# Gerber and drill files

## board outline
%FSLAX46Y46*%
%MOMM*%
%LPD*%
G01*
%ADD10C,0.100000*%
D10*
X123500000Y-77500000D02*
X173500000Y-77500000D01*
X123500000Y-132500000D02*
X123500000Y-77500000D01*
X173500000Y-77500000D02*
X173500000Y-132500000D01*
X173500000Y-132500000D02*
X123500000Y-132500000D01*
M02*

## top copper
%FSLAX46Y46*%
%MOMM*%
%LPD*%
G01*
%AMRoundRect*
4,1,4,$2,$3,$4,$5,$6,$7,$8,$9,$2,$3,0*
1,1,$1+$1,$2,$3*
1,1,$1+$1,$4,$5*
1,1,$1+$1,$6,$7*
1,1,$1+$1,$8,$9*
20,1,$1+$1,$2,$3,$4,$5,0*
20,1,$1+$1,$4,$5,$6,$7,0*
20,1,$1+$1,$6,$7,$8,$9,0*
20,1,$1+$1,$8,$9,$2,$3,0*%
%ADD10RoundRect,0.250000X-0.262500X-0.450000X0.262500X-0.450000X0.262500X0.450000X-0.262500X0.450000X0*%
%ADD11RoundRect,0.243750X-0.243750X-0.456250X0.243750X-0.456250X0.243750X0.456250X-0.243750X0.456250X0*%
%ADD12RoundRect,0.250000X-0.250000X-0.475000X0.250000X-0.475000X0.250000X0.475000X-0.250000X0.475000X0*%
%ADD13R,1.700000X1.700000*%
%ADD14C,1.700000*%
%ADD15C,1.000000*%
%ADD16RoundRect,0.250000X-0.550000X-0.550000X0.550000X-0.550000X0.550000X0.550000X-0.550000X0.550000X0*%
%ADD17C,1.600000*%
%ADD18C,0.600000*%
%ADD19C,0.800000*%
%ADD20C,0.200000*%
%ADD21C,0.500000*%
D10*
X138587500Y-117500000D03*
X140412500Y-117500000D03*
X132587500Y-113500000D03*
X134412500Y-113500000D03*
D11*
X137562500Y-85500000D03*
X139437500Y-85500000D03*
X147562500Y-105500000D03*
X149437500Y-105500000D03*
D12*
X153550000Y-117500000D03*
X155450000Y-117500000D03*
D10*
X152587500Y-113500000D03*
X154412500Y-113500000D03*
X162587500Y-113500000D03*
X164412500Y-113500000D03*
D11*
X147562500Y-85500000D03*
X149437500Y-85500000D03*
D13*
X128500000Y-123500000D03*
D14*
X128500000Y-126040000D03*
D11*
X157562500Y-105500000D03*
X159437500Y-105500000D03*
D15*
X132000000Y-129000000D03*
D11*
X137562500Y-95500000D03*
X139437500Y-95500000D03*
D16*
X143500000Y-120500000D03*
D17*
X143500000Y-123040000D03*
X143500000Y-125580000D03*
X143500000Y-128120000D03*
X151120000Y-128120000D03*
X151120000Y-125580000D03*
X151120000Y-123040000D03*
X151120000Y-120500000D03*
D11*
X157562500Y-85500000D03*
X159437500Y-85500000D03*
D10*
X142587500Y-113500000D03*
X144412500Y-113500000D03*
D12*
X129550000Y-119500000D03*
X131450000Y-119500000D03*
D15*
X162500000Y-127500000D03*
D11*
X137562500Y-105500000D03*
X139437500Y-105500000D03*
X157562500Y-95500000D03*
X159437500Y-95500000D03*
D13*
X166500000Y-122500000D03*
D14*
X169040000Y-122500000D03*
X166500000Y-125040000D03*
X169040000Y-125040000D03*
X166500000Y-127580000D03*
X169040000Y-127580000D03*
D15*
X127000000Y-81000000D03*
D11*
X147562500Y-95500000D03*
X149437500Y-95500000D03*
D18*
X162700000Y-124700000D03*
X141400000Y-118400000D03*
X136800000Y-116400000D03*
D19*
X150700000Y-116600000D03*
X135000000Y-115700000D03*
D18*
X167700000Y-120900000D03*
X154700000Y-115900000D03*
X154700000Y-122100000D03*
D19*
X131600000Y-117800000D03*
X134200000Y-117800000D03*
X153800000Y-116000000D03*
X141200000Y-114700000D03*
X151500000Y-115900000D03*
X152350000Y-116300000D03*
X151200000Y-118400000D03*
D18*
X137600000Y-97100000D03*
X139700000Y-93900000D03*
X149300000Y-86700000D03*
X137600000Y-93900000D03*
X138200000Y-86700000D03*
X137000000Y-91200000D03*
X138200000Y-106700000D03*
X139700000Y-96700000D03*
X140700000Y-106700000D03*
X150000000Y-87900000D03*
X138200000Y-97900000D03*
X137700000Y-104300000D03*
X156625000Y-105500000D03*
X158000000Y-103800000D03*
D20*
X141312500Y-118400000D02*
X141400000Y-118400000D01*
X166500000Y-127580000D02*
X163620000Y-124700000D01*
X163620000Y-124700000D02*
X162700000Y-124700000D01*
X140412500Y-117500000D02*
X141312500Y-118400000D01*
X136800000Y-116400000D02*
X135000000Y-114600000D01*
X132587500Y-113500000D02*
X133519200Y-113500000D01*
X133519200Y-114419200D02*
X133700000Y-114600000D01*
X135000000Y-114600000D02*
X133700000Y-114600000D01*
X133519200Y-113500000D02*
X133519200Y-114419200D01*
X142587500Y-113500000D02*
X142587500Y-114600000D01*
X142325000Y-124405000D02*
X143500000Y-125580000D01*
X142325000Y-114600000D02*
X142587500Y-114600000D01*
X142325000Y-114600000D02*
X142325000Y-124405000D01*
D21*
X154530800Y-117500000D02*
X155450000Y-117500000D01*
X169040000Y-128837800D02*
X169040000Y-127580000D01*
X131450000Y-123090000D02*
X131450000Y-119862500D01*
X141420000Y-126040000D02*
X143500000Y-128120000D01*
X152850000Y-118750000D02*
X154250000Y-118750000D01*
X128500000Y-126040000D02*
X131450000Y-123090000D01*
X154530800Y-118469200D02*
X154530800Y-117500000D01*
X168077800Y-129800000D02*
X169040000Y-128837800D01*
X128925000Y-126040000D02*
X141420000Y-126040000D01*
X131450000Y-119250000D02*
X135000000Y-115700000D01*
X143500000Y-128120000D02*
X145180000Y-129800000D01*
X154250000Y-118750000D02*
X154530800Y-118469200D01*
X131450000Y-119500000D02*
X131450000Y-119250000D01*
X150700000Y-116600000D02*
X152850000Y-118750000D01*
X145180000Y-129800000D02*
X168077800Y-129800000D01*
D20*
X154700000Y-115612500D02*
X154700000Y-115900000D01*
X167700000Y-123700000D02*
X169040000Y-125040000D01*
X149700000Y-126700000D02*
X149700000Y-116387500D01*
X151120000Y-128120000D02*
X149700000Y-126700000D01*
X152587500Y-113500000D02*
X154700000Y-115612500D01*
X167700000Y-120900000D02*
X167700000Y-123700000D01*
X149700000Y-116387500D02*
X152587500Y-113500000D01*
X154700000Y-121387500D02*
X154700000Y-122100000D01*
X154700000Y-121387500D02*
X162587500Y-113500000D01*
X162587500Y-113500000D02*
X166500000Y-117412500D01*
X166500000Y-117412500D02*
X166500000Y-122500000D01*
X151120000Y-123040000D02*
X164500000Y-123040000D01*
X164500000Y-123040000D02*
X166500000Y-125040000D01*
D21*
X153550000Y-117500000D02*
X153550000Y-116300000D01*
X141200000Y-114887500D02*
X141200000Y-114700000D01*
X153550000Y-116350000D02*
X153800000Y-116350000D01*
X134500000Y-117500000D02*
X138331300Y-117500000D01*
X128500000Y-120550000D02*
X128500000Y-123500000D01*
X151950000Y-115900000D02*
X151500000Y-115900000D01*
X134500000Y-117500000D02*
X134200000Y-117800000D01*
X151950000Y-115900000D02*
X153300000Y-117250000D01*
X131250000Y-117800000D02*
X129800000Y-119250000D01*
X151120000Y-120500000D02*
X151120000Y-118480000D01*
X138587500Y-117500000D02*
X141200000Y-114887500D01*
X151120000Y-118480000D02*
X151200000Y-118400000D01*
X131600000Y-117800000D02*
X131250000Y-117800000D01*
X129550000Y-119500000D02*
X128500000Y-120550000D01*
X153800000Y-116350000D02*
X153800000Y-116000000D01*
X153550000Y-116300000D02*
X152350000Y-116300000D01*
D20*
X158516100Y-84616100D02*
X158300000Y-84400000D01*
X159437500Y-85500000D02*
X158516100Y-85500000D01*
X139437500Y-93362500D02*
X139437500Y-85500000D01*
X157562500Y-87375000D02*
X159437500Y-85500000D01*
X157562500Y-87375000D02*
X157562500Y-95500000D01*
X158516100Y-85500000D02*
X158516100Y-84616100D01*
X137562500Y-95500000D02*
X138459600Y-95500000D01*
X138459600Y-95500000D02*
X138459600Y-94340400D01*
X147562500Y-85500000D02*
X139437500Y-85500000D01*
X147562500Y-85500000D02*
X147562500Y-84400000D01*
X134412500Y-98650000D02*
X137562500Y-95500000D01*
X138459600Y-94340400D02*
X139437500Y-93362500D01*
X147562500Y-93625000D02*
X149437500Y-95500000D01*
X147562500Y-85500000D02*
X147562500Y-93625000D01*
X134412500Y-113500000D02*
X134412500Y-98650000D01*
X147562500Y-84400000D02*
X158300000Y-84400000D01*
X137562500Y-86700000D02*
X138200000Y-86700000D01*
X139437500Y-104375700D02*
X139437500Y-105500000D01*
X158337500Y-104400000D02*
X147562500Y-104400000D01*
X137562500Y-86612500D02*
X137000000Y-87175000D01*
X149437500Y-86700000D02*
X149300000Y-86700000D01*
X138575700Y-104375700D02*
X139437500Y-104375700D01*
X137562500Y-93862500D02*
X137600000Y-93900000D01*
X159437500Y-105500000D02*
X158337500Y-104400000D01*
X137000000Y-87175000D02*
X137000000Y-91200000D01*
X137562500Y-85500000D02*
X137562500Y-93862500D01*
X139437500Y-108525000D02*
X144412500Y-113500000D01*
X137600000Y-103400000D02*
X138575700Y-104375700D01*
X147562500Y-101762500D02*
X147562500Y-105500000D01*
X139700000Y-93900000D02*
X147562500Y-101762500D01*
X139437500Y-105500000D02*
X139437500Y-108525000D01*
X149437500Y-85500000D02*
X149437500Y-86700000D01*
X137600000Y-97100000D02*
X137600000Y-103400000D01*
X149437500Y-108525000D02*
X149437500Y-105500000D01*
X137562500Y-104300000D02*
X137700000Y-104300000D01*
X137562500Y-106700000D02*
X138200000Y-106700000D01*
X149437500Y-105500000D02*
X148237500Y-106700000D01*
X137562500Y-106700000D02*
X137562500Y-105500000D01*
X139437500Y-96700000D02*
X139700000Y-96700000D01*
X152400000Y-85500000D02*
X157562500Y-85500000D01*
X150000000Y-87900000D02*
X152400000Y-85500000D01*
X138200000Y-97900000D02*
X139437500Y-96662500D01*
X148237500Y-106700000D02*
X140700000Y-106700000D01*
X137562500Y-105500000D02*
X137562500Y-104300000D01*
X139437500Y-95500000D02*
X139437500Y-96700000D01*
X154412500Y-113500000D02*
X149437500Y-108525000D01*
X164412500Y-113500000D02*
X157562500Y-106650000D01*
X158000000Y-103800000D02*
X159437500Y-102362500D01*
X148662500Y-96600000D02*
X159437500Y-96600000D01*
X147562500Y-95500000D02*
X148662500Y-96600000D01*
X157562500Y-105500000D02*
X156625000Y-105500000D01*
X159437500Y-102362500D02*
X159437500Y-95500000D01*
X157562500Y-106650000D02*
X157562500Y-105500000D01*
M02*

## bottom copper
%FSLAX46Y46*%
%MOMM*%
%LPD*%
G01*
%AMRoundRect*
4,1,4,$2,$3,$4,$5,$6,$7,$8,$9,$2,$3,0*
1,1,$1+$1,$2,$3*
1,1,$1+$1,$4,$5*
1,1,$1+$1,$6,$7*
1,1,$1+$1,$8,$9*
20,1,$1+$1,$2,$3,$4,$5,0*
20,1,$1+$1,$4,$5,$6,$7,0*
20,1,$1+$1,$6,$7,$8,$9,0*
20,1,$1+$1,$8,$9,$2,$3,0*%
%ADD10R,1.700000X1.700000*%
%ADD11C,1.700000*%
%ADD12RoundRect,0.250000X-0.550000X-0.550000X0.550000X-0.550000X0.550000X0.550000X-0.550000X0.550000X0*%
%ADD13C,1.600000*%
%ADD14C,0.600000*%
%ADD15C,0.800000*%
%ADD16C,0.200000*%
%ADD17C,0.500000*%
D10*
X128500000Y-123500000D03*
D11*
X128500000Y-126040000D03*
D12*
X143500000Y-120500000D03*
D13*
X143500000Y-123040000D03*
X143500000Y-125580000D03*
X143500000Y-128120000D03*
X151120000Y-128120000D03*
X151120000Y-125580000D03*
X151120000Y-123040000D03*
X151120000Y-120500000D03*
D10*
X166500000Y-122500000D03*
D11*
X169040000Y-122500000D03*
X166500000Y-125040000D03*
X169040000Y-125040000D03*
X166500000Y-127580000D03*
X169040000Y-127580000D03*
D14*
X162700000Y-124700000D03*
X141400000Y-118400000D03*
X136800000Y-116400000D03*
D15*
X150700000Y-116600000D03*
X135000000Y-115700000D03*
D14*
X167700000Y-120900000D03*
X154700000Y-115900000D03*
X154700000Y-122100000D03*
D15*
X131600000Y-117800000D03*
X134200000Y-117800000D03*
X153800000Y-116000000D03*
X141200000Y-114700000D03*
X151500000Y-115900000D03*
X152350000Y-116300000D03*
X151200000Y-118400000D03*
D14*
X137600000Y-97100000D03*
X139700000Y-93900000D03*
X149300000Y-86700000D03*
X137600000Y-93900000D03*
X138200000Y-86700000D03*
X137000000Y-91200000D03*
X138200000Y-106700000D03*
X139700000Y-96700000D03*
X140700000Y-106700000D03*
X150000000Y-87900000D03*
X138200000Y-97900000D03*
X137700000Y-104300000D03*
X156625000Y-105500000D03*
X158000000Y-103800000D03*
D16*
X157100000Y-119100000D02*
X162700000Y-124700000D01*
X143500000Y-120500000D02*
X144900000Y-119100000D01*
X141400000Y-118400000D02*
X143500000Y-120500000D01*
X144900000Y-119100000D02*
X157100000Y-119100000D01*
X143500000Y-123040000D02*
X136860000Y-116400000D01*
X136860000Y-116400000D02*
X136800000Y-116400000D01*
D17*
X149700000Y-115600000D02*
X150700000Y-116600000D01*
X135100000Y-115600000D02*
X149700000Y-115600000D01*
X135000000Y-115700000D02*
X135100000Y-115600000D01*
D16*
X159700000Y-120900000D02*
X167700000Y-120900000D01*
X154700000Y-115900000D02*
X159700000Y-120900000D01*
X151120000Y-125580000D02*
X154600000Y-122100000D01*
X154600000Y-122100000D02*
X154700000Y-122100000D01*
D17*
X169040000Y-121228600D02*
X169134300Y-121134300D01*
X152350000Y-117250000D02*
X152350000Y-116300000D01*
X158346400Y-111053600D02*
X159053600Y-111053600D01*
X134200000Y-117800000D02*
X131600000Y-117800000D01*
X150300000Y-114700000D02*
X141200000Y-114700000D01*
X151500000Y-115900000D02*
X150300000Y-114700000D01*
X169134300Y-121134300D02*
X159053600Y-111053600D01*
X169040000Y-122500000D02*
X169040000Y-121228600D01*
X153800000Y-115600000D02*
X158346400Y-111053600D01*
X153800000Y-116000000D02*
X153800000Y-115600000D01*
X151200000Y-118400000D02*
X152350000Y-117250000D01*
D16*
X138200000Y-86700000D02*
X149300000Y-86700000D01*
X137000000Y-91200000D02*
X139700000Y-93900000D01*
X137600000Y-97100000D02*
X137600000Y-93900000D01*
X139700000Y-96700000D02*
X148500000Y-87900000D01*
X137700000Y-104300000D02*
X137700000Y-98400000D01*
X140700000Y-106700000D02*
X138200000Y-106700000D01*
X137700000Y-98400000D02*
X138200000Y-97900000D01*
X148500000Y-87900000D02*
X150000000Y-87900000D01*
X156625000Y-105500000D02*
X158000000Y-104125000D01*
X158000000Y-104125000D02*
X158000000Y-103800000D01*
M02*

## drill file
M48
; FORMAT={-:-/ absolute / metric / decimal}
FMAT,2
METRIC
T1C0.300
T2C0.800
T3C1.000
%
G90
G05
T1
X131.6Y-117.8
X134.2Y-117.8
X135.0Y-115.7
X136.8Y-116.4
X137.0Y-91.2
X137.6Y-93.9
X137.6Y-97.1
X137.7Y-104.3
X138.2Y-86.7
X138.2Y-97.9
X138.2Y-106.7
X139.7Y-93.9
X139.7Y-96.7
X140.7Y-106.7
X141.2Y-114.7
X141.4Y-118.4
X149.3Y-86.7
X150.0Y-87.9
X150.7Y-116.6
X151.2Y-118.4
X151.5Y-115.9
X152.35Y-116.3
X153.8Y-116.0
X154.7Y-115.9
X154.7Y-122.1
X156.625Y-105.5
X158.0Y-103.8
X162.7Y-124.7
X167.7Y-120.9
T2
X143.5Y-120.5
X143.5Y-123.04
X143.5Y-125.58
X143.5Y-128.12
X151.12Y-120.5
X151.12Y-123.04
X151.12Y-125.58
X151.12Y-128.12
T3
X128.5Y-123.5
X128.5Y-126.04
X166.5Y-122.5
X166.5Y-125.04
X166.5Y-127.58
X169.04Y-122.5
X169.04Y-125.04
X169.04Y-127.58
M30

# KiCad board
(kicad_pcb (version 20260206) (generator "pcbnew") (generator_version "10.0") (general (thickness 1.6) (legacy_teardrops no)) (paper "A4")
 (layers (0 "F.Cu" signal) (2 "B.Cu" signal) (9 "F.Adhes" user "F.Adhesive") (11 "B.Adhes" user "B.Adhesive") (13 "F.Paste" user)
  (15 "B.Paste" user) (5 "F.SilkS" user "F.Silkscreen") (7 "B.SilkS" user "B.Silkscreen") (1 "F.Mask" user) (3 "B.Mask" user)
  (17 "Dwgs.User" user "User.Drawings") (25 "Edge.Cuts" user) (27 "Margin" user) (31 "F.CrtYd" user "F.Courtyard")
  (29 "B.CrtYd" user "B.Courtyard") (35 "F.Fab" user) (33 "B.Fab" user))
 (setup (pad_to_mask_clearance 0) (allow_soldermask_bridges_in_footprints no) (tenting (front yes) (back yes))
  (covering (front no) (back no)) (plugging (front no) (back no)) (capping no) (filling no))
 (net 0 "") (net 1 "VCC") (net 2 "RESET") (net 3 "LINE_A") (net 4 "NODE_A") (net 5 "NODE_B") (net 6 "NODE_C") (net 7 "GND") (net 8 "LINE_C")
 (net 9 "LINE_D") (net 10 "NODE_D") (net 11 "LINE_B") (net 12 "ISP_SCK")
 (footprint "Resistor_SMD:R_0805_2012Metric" (layer "F.Cu") (at 139.5 117.5)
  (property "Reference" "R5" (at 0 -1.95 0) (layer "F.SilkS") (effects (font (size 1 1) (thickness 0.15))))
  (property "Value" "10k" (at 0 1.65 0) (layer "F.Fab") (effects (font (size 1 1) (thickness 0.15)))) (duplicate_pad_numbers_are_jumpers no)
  (pad "1" smd roundrect (at -0.9125 0) (size 1.025 1.4) (layers "F.Cu" "F.Mask" "F.Paste") (roundrect_rratio 0.243902) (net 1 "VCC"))
  (pad "2" smd roundrect (at 0.9125 0) (size 1.025 1.4) (layers "F.Cu" "F.Mask" "F.Paste") (roundrect_rratio 0.243902) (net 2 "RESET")))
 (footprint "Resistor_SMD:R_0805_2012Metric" (layer "F.Cu") (at 133.5 113.5)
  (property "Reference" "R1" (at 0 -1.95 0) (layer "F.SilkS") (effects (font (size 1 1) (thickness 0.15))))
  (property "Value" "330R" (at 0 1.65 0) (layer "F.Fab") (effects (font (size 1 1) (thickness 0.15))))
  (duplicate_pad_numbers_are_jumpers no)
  (pad "1" smd roundrect (at -0.9125 0) (size 1.025 1.4) (layers "F.Cu" "F.Mask" "F.Paste") (roundrect_rratio 0.243902) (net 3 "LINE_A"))
  (pad "2" smd roundrect (at 0.9125 0) (size 1.025 1.4) (layers "F.Cu" "F.Mask" "F.Paste") (roundrect_rratio 0.243902) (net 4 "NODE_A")))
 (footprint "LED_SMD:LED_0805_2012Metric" (layer "F.Cu") (at 138.5 85.5)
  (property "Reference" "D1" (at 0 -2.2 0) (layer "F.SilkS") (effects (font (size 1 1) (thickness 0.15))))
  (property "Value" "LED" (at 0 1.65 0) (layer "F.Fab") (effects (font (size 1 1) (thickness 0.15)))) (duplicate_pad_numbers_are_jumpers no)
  (pad "1" smd roundrect (at -0.9375 0) (size 0.975 1.4) (layers "F.Cu" "F.Mask" "F.Paste") (roundrect_rratio 0.25) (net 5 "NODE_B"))
  (pad "2" smd roundrect (at 0.9375 0) (size 0.975 1.4) (layers "F.Cu" "F.Mask" "F.Paste") (roundrect_rratio 0.25) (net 4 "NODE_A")))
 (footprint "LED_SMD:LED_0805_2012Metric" (layer "F.Cu") (at 148.5 105.5)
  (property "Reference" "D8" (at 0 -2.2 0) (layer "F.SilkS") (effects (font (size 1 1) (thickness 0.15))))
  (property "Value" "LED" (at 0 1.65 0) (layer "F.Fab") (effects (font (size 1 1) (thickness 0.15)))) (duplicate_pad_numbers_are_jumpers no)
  (pad "1" smd roundrect (at -0.9375 0) (size 0.975 1.4) (layers "F.Cu" "F.Mask" "F.Paste") (roundrect_rratio 0.25) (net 5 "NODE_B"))
  (pad "2" smd roundrect (at 0.9375 0) (size 0.975 1.4) (layers "F.Cu" "F.Mask" "F.Paste") (roundrect_rratio 0.25) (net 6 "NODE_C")))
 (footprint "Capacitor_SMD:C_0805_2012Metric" (layer "F.Cu") (at 154.5 117.5)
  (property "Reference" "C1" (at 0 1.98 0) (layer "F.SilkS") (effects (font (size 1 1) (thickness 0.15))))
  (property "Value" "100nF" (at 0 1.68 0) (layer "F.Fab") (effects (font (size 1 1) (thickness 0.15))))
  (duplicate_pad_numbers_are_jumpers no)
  (pad "1" smd roundrect (at -0.95 0) (size 1 1.45) (layers "F.Cu" "F.Mask" "F.Paste") (roundrect_rratio 0.25) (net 1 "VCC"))
  (pad "2" smd roundrect (at 0.95 0) (size 1 1.45) (layers "F.Cu" "F.Mask" "F.Paste") (roundrect_rratio 0.25) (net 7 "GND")))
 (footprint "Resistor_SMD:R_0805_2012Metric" (layer "F.Cu") (at 153.5 113.5)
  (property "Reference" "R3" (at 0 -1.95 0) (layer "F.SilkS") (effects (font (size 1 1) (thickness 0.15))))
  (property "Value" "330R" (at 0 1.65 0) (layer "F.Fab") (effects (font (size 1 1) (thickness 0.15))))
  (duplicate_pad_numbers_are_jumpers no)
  (pad "1" smd roundrect (at -0.9125 0) (size 1.025 1.4) (layers "F.Cu" "F.Mask" "F.Paste") (roundrect_rratio 0.243902) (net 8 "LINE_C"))
  (pad "2" smd roundrect (at 0.9125 0) (size 1.025 1.4) (layers "F.Cu" "F.Mask" "F.Paste") (roundrect_rratio 0.243902) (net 6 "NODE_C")))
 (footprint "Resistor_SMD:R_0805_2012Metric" (layer "F.Cu") (at 163.5 113.5)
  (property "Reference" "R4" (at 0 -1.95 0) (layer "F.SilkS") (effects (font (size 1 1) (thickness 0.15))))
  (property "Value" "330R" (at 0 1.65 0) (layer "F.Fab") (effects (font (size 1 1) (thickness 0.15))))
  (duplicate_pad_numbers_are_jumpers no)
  (pad "1" smd roundrect (at -0.9125 0) (size 1.025 1.4) (layers "F.Cu" "F.Mask" "F.Paste") (roundrect_rratio 0.243902) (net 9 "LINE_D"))
  (pad "2" smd roundrect (at 0.9125 0) (size 1.025 1.4) (layers "F.Cu" "F.Mask" "F.Paste") (roundrect_rratio 0.243902) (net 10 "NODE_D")))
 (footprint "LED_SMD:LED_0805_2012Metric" (layer "F.Cu") (at 148.5 85.5)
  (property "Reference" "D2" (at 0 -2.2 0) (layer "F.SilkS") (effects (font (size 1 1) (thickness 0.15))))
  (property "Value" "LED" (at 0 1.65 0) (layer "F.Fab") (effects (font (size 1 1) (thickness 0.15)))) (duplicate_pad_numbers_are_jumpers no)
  (pad "1" smd roundrect (at -0.9375 0) (size 0.975 1.4) (layers "F.Cu" "F.Mask" "F.Paste") (roundrect_rratio 0.25) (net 4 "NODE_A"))
  (pad "2" smd roundrect (at 0.9375 0) (size 0.975 1.4) (layers "F.Cu" "F.Mask" "F.Paste") (roundrect_rratio 0.25) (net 5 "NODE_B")))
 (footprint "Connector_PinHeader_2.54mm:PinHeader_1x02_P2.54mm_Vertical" (layer "F.Cu") (at 128.5 123.5)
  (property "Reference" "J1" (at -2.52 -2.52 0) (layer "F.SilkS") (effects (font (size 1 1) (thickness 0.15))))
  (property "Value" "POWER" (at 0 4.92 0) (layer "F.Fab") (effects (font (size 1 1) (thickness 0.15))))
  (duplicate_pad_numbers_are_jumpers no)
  (pad "1" thru_hole rect (at 0 0) (size 1.7 1.7) (drill 1) (layers "*.Cu" "*.Mask") (remove_unused_layers no) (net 1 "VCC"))
  (pad "2" thru_hole circle (at 0 2.54) (size 1.7 1.7) (drill 1) (layers "*.Cu" "*.Mask") (remove_unused_layers no) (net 7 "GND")))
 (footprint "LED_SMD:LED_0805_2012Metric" (layer "F.Cu") (at 158.5 105.5)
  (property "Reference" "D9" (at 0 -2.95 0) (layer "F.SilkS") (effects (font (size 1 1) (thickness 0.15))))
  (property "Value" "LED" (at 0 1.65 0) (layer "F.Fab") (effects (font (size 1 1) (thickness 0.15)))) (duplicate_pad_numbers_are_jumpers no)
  (pad "1" smd roundrect (at -0.9375 0) (size 0.975 1.4) (layers "F.Cu" "F.Mask" "F.Paste") (roundrect_rratio 0.25) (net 10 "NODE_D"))
  (pad "2" smd roundrect (at 0.9375 0) (size 0.975 1.4) (layers "F.Cu" "F.Mask" "F.Paste") (roundrect_rratio 0.25) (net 5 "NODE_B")))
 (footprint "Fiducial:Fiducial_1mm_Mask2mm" (layer "F.Cu") (at 132 129)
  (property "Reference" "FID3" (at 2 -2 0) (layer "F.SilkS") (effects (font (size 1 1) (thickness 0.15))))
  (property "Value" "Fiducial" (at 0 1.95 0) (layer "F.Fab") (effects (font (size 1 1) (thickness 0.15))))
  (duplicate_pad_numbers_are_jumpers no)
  (pad "" smd circle (at 0 0) (size 1 1) (layers "F.Cu" "F.Mask") (solder_mask_margin 0.5) (clearance 0.6)))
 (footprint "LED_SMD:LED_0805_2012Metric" (layer "F.Cu") (at 138.5 95.5)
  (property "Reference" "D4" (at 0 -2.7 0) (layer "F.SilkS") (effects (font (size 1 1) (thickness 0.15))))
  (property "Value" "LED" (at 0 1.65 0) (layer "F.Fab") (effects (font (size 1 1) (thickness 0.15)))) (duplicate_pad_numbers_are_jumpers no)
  (pad "1" smd roundrect (at -0.9375 0) (size 0.975 1.4) (layers "F.Cu" "F.Mask" "F.Paste") (roundrect_rratio 0.25) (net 4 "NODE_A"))
  (pad "2" smd roundrect (at 0.9375 0) (size 0.975 1.4) (layers "F.Cu" "F.Mask" "F.Paste") (roundrect_rratio 0.25) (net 6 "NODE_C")))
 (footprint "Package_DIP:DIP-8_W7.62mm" (layer "F.Cu") (at 143.5 120.5)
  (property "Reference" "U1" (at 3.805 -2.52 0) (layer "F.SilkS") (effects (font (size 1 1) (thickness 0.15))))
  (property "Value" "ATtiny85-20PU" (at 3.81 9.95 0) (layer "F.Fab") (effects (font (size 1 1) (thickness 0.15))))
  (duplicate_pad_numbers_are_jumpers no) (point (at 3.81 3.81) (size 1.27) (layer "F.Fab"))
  (pad "1" thru_hole roundrect (at 0 0) (size 1.6 1.6) (drill 0.8) (layers "*.Cu" "*.Mask") (remove_unused_layers no)
   (roundrect_rratio 0.15625) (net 2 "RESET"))
  (pad "2" thru_hole circle (at 0 2.54) (size 1.6 1.6) (drill 0.8) (layers "*.Cu" "*.Mask") (remove_unused_layers no) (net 3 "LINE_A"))
  (pad "3" thru_hole circle (at 0 5.08) (size 1.6 1.6) (drill 0.8) (layers "*.Cu" "*.Mask") (remove_unused_layers no) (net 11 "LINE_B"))
  (pad "4" thru_hole circle (at 0 7.62) (size 1.6 1.6) (drill 0.8) (layers "*.Cu" "*.Mask") (remove_unused_layers no) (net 7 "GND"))
  (pad "5" thru_hole circle (at 7.62 7.62) (size 1.6 1.6) (drill 0.8) (layers "*.Cu" "*.Mask") (remove_unused_layers no) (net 8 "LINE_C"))
  (pad "6" thru_hole circle (at 7.62 5.08) (size 1.6 1.6) (drill 0.8) (layers "*.Cu" "*.Mask") (remove_unused_layers no) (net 9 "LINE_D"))
  (pad "7" thru_hole circle (at 7.62 2.54) (size 1.6 1.6) (drill 0.8) (layers "*.Cu" "*.Mask") (remove_unused_layers no) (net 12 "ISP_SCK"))
  (pad "8" thru_hole circle (at 7.62 0) (size 1.6 1.6) (drill 0.8) (layers "*.Cu" "*.Mask") (remove_unused_layers no) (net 1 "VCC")))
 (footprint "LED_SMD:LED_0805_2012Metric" (layer "F.Cu") (at 158.5 85.5)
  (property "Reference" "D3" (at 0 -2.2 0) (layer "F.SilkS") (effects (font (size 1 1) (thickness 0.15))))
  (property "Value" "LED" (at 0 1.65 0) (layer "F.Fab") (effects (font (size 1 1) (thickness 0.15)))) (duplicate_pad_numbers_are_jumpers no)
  (pad "1" smd roundrect (at -0.9375 0) (size 0.975 1.4) (layers "F.Cu" "F.Mask" "F.Paste") (roundrect_rratio 0.25) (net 6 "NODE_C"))
  (pad "2" smd roundrect (at 0.9375 0) (size 0.975 1.4) (layers "F.Cu" "F.Mask" "F.Paste") (roundrect_rratio 0.25) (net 4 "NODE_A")))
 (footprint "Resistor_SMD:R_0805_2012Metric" (layer "F.Cu") (at 143.5 113.5)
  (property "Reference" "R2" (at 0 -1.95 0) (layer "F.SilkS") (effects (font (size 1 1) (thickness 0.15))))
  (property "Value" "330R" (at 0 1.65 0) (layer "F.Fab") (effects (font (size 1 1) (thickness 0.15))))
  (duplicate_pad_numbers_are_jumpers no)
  (pad "1" smd roundrect (at -0.9125 0) (size 1.025 1.4) (layers "F.Cu" "F.Mask" "F.Paste") (roundrect_rratio 0.243902) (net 11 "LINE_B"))
  (pad "2" smd roundrect (at 0.9125 0) (size 1.025 1.4) (layers "F.Cu" "F.Mask" "F.Paste") (roundrect_rratio 0.243902) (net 5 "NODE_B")))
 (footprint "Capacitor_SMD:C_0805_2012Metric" (layer "F.Cu") (at 130.5 119.5)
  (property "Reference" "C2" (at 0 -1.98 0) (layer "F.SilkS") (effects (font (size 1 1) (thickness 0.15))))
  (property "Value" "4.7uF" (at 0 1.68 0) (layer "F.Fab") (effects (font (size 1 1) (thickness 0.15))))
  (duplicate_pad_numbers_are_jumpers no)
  (pad "1" smd roundrect (at -0.95 0) (size 1 1.45) (layers "F.Cu" "F.Mask" "F.Paste") (roundrect_rratio 0.25) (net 1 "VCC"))
  (pad "2" smd roundrect (at 0.95 0) (size 1 1.45) (layers "F.Cu" "F.Mask" "F.Paste") (roundrect_rratio 0.25) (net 7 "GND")))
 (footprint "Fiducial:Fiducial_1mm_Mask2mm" (layer "F.Cu") (at 162.5 127.5)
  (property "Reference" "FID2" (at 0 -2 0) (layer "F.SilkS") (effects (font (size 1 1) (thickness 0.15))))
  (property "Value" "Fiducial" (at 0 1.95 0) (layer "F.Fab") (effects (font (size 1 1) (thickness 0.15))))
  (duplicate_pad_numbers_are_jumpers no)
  (pad "" smd circle (at 0 0) (size 1 1) (layers "F.Cu" "F.Mask") (solder_mask_margin 0.5) (clearance 0.6)))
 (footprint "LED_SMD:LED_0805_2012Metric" (layer "F.Cu") (at 138.5 105.5)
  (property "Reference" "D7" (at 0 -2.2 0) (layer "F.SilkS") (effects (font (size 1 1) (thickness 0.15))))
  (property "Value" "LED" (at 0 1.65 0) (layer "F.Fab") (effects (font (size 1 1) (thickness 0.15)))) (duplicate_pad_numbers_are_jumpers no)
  (pad "1" smd roundrect (at -0.9375 0) (size 0.975 1.4) (layers "F.Cu" "F.Mask" "F.Paste") (roundrect_rratio 0.25) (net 6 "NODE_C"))
  (pad "2" smd roundrect (at 0.9375 0) (size 0.975 1.4) (layers "F.Cu" "F.Mask" "F.Paste") (roundrect_rratio 0.25) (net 5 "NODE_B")))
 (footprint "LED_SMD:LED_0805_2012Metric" (layer "F.Cu") (at 158.5 95.5)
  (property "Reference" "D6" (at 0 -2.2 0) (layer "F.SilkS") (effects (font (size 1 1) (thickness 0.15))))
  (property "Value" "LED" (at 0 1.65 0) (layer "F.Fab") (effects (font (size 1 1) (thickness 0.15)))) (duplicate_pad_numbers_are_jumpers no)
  (pad "1" smd roundrect (at -0.9375 0) (size 0.975 1.4) (layers "F.Cu" "F.Mask" "F.Paste") (roundrect_rratio 0.25) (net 4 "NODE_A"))
  (pad "2" smd roundrect (at 0.9375 0) (size 0.975 1.4) (layers "F.Cu" "F.Mask" "F.Paste") (roundrect_rratio 0.25) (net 10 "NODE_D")))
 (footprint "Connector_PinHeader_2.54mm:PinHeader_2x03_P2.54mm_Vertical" (layer "F.Cu") (at 166.5 122.5)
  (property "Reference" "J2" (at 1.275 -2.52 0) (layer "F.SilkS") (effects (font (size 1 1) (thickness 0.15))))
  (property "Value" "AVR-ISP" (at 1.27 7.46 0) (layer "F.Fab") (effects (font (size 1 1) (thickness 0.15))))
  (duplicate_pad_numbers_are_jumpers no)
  (pad "1" thru_hole rect (at 0 0) (size 1.7 1.7) (drill 1) (layers "*.Cu" "*.Mask") (remove_unused_layers no) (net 9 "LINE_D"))
  (pad "2" thru_hole circle (at 2.54 0) (size 1.7 1.7) (drill 1) (layers "*.Cu" "*.Mask") (remove_unused_layers no) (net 1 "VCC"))
  (pad "3" thru_hole circle (at 0 2.54) (size 1.7 1.7) (drill 1) (layers "*.Cu" "*.Mask") (remove_unused_layers no) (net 12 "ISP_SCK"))
  (pad "4" thru_hole circle (at 2.54 2.54) (size 1.7 1.7) (drill 1) (layers "*.Cu" "*.Mask") (remove_unused_layers no) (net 8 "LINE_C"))
  (pad "5" thru_hole circle (at 0 5.08) (size 1.7 1.7) (drill 1) (layers "*.Cu" "*.Mask") (remove_unused_layers no) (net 2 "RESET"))
  (pad "6" thru_hole circle (at 2.54 5.08) (size 1.7 1.7) (drill 1) (layers "*.Cu" "*.Mask") (remove_unused_layers no) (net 7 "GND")))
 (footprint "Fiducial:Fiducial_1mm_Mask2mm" (layer "F.Cu") (at 127 81)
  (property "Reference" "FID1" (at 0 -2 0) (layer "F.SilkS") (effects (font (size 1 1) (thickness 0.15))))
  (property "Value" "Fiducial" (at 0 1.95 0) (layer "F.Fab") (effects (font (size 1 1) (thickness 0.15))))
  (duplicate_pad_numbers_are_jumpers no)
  (pad "" smd circle (at 0 0) (size 1 1) (layers "F.Cu" "F.Mask") (solder_mask_margin 0.5) (clearance 0.6)))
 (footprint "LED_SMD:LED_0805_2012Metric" (layer "F.Cu") (at 148.5 95.5)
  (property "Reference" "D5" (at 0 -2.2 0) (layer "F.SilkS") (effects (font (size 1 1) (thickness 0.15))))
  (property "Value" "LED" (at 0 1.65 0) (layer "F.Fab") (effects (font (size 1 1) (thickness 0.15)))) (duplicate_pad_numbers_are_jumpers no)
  (pad "1" smd roundrect (at -0.9375 0) (size 0.975 1.4) (layers "F.Cu" "F.Mask" "F.Paste") (roundrect_rratio 0.25) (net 10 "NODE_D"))
  (pad "2" smd roundrect (at 0.9375 0) (size 0.975 1.4) (layers "F.Cu" "F.Mask" "F.Paste") (roundrect_rratio 0.25) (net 4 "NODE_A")))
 (gr_line (start 123.5 77.5) (end 173.5 77.5) (stroke (width 0.1) (type default)) (layer "Edge.Cuts"))
 (gr_line (start 123.5 132.5) (end 123.5 77.5) (stroke (width 0.1) (type default)) (layer "Edge.Cuts"))
 (gr_line (start 173.5 77.5) (end 173.5 132.5) (stroke (width 0.1) (type default)) (layer "Edge.Cuts"))
 (gr_line (start 173.5 132.5) (end 123.5 132.5) (stroke (width 0.1) (type default)) (layer "Edge.Cuts"))
 (segment (start 141.3125 118.4) (end 141.4 118.4) (width 0.2) (layer "F.Cu") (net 2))
 (segment (start 166.5 127.58) (end 163.62 124.7) (width 0.2) (layer "F.Cu") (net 2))
 (segment (start 163.62 124.7) (end 162.7 124.7) (width 0.2) (layer "F.Cu") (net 2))
 (segment (start 140.4125 117.5) (end 141.3125 118.4) (width 0.2) (layer "F.Cu") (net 2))
 (via (at 162.7 124.7) (size 0.6) (drill 0.3) (layers "F.Cu" "B.Cu") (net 2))
 (via (at 141.4 118.4) (size 0.6) (drill 0.3) (layers "F.Cu" "B.Cu") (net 2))
 (segment (start 157.1 119.1) (end 162.7 124.7) (width 0.2) (layer "B.Cu") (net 2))
 (segment (start 143.5 120.5) (end 144.9 119.1) (width 0.2) (layer "B.Cu") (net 2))
 (segment (start 141.4 118.4) (end 143.5 120.5) (width 0.2) (layer "B.Cu") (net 2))
 (segment (start 144.9 119.1) (end 157.1 119.1) (width 0.2) (layer "B.Cu") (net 2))
 (segment (start 136.8 116.4) (end 135 114.6) (width 0.2) (layer "F.Cu") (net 3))
 (segment (start 132.5875 113.5) (end 133.5192 113.5) (width 0.2) (layer "F.Cu") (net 3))
 (segment (start 133.5192 114.4192) (end 133.7 114.6) (width 0.2) (layer "F.Cu") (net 3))
 (segment (start 135 114.6) (end 133.7 114.6) (width 0.2) (layer "F.Cu") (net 3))
 (segment (start 133.5192 113.5) (end 133.5192 114.4192) (width 0.2) (layer "F.Cu") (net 3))
 (via (at 136.8 116.4) (size 0.6) (drill 0.3) (layers "F.Cu" "B.Cu") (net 3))
 (segment (start 143.5 123.04) (end 136.86 116.4) (width 0.2) (layer "B.Cu") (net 3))
 (segment (start 136.86 116.4) (end 136.8 116.4) (width 0.2) (layer "B.Cu") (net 3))
 (segment (start 142.5875 113.5) (end 142.5875 114.6) (width 0.2) (layer "F.Cu") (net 11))
 (segment (start 142.325 124.405) (end 143.5 125.58) (width 0.2) (layer "F.Cu") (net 11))
 (segment (start 142.325 114.6) (end 142.5875 114.6) (width 0.2) (layer "F.Cu") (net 11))
 (segment (start 142.325 114.6) (end 142.325 124.405) (width 0.2) (layer "F.Cu") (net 11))
 (segment (start 154.5308 117.5) (end 155.45 117.5) (width 0.5) (layer "F.Cu") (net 7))
 (segment (start 169.04 128.8378) (end 169.04 127.58) (width 0.5) (layer "F.Cu") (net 7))
 (segment (start 131.45 123.09) (end 131.45 119.8625) (width 0.5) (layer "F.Cu") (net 7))
 (segment (start 141.42 126.04) (end 143.5 128.12) (width 0.5) (layer "F.Cu") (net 7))
 (segment (start 152.85 118.75) (end 154.25 118.75) (width 0.5) (layer "F.Cu") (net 7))
 (segment (start 128.5 126.04) (end 131.45 123.09) (width 0.5) (layer "F.Cu") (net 7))
 (segment (start 154.5308 118.4692) (end 154.5308 117.5) (width 0.5) (layer "F.Cu") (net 7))
 (segment (start 168.0778 129.8) (end 169.04 128.8378) (width 0.5) (layer "F.Cu") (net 7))
 (segment (start 128.925 126.04) (end 141.42 126.04) (width 0.5) (layer "F.Cu") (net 7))
 (segment (start 131.45 119.25) (end 135 115.7) (width 0.5) (layer "F.Cu") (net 7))
 (segment (start 143.5 128.12) (end 145.18 129.8) (width 0.5) (layer "F.Cu") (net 7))
 (segment (start 154.25 118.75) (end 154.5308 118.4692) (width 0.5) (layer "F.Cu") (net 7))
 (segment (start 131.45 119.5) (end 131.45 119.25) (width 0.5) (layer "F.Cu") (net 7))
 (segment (start 150.7 116.6) (end 152.85 118.75) (width 0.5) (layer "F.Cu") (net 7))
 (segment (start 145.18 129.8) (end 168.0778 129.8) (width 0.5) (layer "F.Cu") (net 7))
 (via (at 150.7 116.6) (size 0.8) (drill 0.3) (layers "F.Cu" "B.Cu") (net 7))
 (via (at 135 115.7) (size 0.8) (drill 0.3) (layers "F.Cu" "B.Cu") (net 7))
 (segment (start 149.7 115.6) (end 150.7 116.6) (width 0.5) (layer "B.Cu") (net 7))
 (segment (start 135.1 115.6) (end 149.7 115.6) (width 0.5) (layer "B.Cu") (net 7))
 (segment (start 135 115.7) (end 135.1 115.6) (width 0.5) (layer "B.Cu") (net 7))
 (segment (start 154.7 115.6125) (end 154.7 115.9) (width 0.2) (layer "F.Cu") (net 8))
 (segment (start 167.7 123.7) (end 169.04 125.04) (width 0.2) (layer "F.Cu") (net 8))
 (segment (start 149.7 126.7) (end 149.7 116.3875) (width 0.2) (layer "F.Cu") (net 8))
 (segment (start 151.12 128.12) (end 149.7 126.7) (width 0.2) (layer "F.Cu") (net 8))
 (segment (start 152.5875 113.5) (end 154.7 115.6125) (width 0.2) (layer "F.Cu") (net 8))
 (segment (start 167.7 120.9) (end 167.7 123.7) (width 0.2) (layer "F.Cu") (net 8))
 (segment (start 149.7 116.3875) (end 152.5875 113.5) (width 0.2) (layer "F.Cu") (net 8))
 (via (at 167.7 120.9) (size 0.6) (drill 0.3) (layers "F.Cu" "B.Cu") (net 8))
 (via (at 154.7 115.9) (size 0.6) (drill 0.3) (layers "F.Cu" "B.Cu") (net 8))
 (segment (start 159.7 120.9) (end 167.7 120.9) (width 0.2) (layer "B.Cu") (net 8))
 (segment (start 154.7 115.9) (end 159.7 120.9) (width 0.2) (layer "B.Cu") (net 8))
 (segment (start 154.7 121.3875) (end 154.7 122.1) (width 0.2) (layer "F.Cu") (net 9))
 (segment (start 154.7 121.3875) (end 162.5875 113.5) (width 0.2) (layer "F.Cu") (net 9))
 (segment (start 162.5875 113.5) (end 166.5 117.4125) (width 0.2) (layer "F.Cu") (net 9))
 (segment (start 166.5 117.4125) (end 166.5 122.5) (width 0.2) (layer "F.Cu") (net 9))
 (via (at 154.7 122.1) (size 0.6) (drill 0.3) (layers "F.Cu" "B.Cu") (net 9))
 (segment (start 151.12 125.58) (end 154.6 122.1) (width 0.2) (layer "B.Cu") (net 9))
 (segment (start 154.6 122.1) (end 154.7 122.1) (width 0.2) (layer "B.Cu") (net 9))
 (segment (start 151.12 123.04) (end 164.5 123.04) (width 0.2) (layer "F.Cu") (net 12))
 (segment (start 164.5 123.04) (end 166.5 125.04) (width 0.2) (layer "F.Cu") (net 12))
 (segment (start 153.55 117.5) (end 153.55 116.3) (width 0.5) (layer "F.Cu") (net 1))
 (segment (start 141.2 114.8875) (end 141.2 114.7) (width 0.5) (layer "F.Cu") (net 1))
 (segment (start 153.55 116.35) (end 153.8 116.35) (width 0.5) (layer "F.Cu") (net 1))
 (segment (start 134.5 117.5) (end 138.3313 117.5) (width 0.5) (layer "F.Cu") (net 1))
 (segment (start 128.5 120.55) (end 128.5 123.5) (width 0.5) (layer "F.Cu") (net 1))
 (segment (start 151.95 115.9) (end 151.5 115.9) (width 0.5) (layer "F.Cu") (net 1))
 (segment (start 134.5 117.5) (end 134.2 117.8) (width 0.5) (layer "F.Cu") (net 1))
 (segment (start 151.95 115.9) (end 153.3 117.25) (width 0.5) (layer "F.Cu") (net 1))
 (segment (start 131.25 117.8) (end 129.8 119.25) (width 0.5) (layer "F.Cu") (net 1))
 (segment (start 151.12 120.5) (end 151.12 118.48) (width 0.5) (layer "F.Cu") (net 1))
 (segment (start 138.5875 117.5) (end 141.2 114.8875) (width 0.5) (layer "F.Cu") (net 1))
 (segment (start 151.12 118.48) (end 151.2 118.4) (width 0.5) (layer "F.Cu") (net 1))
 (segment (start 131.6 117.8) (end 131.25 117.8) (width 0.5) (layer "F.Cu") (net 1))
 (segment (start 129.55 119.5) (end 128.5 120.55) (width 0.5) (layer "F.Cu") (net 1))
 (segment (start 153.8 116.35) (end 153.8 116) (width 0.5) (layer "F.Cu") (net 1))
 (segment (start 153.55 116.3) (end 152.35 116.3) (width 0.5) (layer "F.Cu") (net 1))
 (via (at 131.6 117.8) (size 0.8) (drill 0.3) (layers "F.Cu" "B.Cu") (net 1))
 (via (at 134.2 117.8) (size 0.8) (drill 0.3) (layers "F.Cu" "B.Cu") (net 1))
 (via (at 153.8 116) (size 0.8) (drill 0.3) (layers "F.Cu" "B.Cu") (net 1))
 (via (at 141.2 114.7) (size 0.8) (drill 0.3) (layers "F.Cu" "B.Cu") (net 1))
 (via (at 151.5 115.9) (size 0.8) (drill 0.3) (layers "F.Cu" "B.Cu") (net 1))
 (via (at 152.35 116.3) (size 0.8) (drill 0.3) (layers "F.Cu" "B.Cu") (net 1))
 (via (at 151.2 118.4) (size 0.8) (drill 0.3) (layers "F.Cu" "B.Cu") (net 1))
 (segment (start 169.04 121.2286) (end 169.1343 121.1343) (width 0.5) (layer "B.Cu") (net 1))
 (segment (start 152.35 117.25) (end 152.35 116.3) (width 0.5) (layer "B.Cu") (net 1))
 (segment (start 158.3464 111.0536) (end 159.0536 111.0536) (width 0.5) (layer "B.Cu") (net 1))
 (segment (start 134.2 117.8) (end 131.6 117.8) (width 0.5) (layer "B.Cu") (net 1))
 (segment (start 150.3 114.7) (end 141.2 114.7) (width 0.5) (layer "B.Cu") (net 1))
 (segment (start 151.5 115.9) (end 150.3 114.7) (width 0.5) (layer "B.Cu") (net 1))
 (segment (start 169.1343 121.1343) (end 159.0536 111.0536) (width 0.5) (layer "B.Cu") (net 1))
 (segment (start 169.04 122.5) (end 169.04 121.2286) (width 0.5) (layer "B.Cu") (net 1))
 (segment (start 153.8 115.6) (end 158.3464 111.0536) (width 0.5) (layer "B.Cu") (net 1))
 (segment (start 153.8 116) (end 153.8 115.6) (width 0.5) (layer "B.Cu") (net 1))
 (segment (start 151.2 118.4) (end 152.35 117.25) (width 0.5) (layer "B.Cu") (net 1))
 (segment (start 158.5161 84.6161) (end 158.3 84.4) (width 0.2) (layer "F.Cu") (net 4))
 (segment (start 159.4375 85.5) (end 158.5161 85.5) (width 0.2) (layer "F.Cu") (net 4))
 (segment (start 139.4375 93.3625) (end 139.4375 85.5) (width 0.2) (layer "F.Cu") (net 4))
 (segment (start 157.5625 87.375) (end 159.4375 85.5) (width 0.2) (layer "F.Cu") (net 4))
 (segment (start 157.5625 87.375) (end 157.5625 95.5) (width 0.2) (layer "F.Cu") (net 4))
 (segment (start 158.5161 85.5) (end 158.5161 84.6161) (width 0.2) (layer "F.Cu") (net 4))
 (segment (start 137.5625 95.5) (end 138.4596 95.5) (width 0.2) (layer "F.Cu") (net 4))
 (segment (start 138.4596 95.5) (end 138.4596 94.3404) (width 0.2) (layer "F.Cu") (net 4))
 (segment (start 147.5625 85.5) (end 139.4375 85.5) (width 0.2) (layer "F.Cu") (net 4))
 (segment (start 147.5625 85.5) (end 147.5625 84.4) (width 0.2) (layer "F.Cu") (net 4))
 (segment (start 134.4125 98.65) (end 137.5625 95.5) (width 0.2) (layer "F.Cu") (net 4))
 (segment (start 138.4596 94.3404) (end 139.4375 93.3625) (width 0.2) (layer "F.Cu") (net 4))
 (segment (start 147.5625 93.625) (end 149.4375 95.5) (width 0.2) (layer "F.Cu") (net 4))
 (segment (start 147.5625 85.5) (end 147.5625 93.625) (width 0.2) (layer "F.Cu") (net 4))
 (segment (start 134.4125 113.5) (end 134.4125 98.65) (width 0.2) (layer "F.Cu") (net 4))
 (segment (start 147.5625 84.4) (end 158.3 84.4) (width 0.2) (layer "F.Cu") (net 4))
 (segment (start 137.5625 86.7) (end 138.2 86.7) (width 0.2) (layer "F.Cu") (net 5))
 (segment (start 139.4375 104.3757) (end 139.4375 105.5) (width 0.2) (layer "F.Cu") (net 5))
 (segment (start 158.3375 104.4) (end 147.5625 104.4) (width 0.2) (layer "F.Cu") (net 5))
 (segment (start 137.5625 86.6125) (end 137 87.175) (width 0.2) (layer "F.Cu") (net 5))
 (segment (start 149.4375 86.7) (end 149.3 86.7) (width 0.2) (layer "F.Cu") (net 5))
 (segment (start 138.5757 104.3757) (end 139.4375 104.3757) (width 0.2) (layer "F.Cu") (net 5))
 (segment (start 137.5625 93.8625) (end 137.6 93.9) (width 0.2) (layer "F.Cu") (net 5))
 (segment (start 159.4375 105.5) (end 158.3375 104.4) (width 0.2) (layer "F.Cu") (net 5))
 (segment (start 137 87.175) (end 137 91.2) (width 0.2) (layer "F.Cu") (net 5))
 (segment (start 137.5625 85.5) (end 137.5625 93.8625) (width 0.2) (layer "F.Cu") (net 5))
 (segment (start 139.4375 108.525) (end 144.4125 113.5) (width 0.2) (layer "F.Cu") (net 5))
 (segment (start 137.6 103.4) (end 138.5757 104.3757) (width 0.2) (layer "F.Cu") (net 5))
 (segment (start 147.5625 101.7625) (end 147.5625 105.5) (width 0.2) (layer "F.Cu") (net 5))
 (segment (start 139.7 93.9) (end 147.5625 101.7625) (width 0.2) (layer "F.Cu") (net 5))
 (segment (start 139.4375 105.5) (end 139.4375 108.525) (width 0.2) (layer "F.Cu") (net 5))
 (segment (start 149.4375 85.5) (end 149.4375 86.7) (width 0.2) (layer "F.Cu") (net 5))
 (segment (start 137.6 97.1) (end 137.6 103.4) (width 0.2) (layer "F.Cu") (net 5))
 (via (at 137.6 97.1) (size 0.6) (drill 0.3) (layers "F.Cu" "B.Cu") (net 5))
 (via (at 139.7 93.9) (size 0.6) (drill 0.3) (layers "F.Cu" "B.Cu") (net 5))
 (via (at 149.3 86.7) (size 0.6) (drill 0.3) (layers "F.Cu" "B.Cu") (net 5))
 (via (at 137.6 93.9) (size 0.6) (drill 0.3) (layers "F.Cu" "B.Cu") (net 5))
 (via (at 138.2 86.7) (size 0.6) (drill 0.3) (layers "F.Cu" "B.Cu") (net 5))
 (via (at 137 91.2) (size 0.6) (drill 0.3) (layers "F.Cu" "B.Cu") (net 5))
 (segment (start 138.2 86.7) (end 149.3 86.7) (width 0.2) (layer "B.Cu") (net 5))
 (segment (start 137 91.2) (end 139.7 93.9) (width 0.2) (layer "B.Cu") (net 5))
 (segment (start 137.6 97.1) (end 137.6 93.9) (width 0.2) (layer "B.Cu") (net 5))
 (segment (start 149.4375 108.525) (end 149.4375 105.5) (width 0.2) (layer "F.Cu") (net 6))
 (segment (start 137.5625 104.3) (end 137.7 104.3) (width 0.2) (layer "F.Cu") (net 6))
 (segment (start 137.5625 106.7) (end 138.2 106.7) (width 0.2) (layer "F.Cu") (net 6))
 (segment (start 149.4375 105.5) (end 148.2375 106.7) (width 0.2) (layer "F.Cu") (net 6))
 (segment (start 137.5625 106.7) (end 137.5625 105.5) (width 0.2) (layer "F.Cu") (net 6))
 (segment (start 139.4375 96.7) (end 139.7 96.7) (width 0.2) (layer "F.Cu") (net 6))
 (segment (start 152.4 85.5) (end 157.5625 85.5) (width 0.2) (layer "F.Cu") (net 6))
 (segment (start 150 87.9) (end 152.4 85.5) (width 0.2) (layer "F.Cu") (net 6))
 (segment (start 138.2 97.9) (end 139.4375 96.6625) (width 0.2) (layer "F.Cu") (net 6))
 (segment (start 148.2375 106.7) (end 140.7 106.7) (width 0.2) (layer "F.Cu") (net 6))
 (segment (start 137.5625 105.5) (end 137.5625 104.3) (width 0.2) (layer "F.Cu") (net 6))
 (segment (start 139.4375 95.5) (end 139.4375 96.7) (width 0.2) (layer "F.Cu") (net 6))
 (segment (start 154.4125 113.5) (end 149.4375 108.525) (width 0.2) (layer "F.Cu") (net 6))
 (via (at 138.2 106.7) (size 0.6) (drill 0.3) (layers "F.Cu" "B.Cu") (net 6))
 (via (at 139.7 96.7) (size 0.6) (drill 0.3) (layers "F.Cu" "B.Cu") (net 6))
 (via (at 140.7 106.7) (size 0.6) (drill 0.3) (layers "F.Cu" "B.Cu") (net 6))
 (via (at 150 87.9) (size 0.6) (drill 0.3) (layers "F.Cu" "B.Cu") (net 6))
 (via (at 138.2 97.9) (size 0.6) (drill 0.3) (layers "F.Cu" "B.Cu") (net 6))
 (via (at 137.7 104.3) (size 0.6) (drill 0.3) (layers "F.Cu" "B.Cu") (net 6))
 (segment (start 139.7 96.7) (end 148.5 87.9) (width 0.2) (layer "B.Cu") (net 6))
 (segment (start 137.7 104.3) (end 137.7 98.4) (width 0.2) (layer "B.Cu") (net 6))
 (segment (start 140.7 106.7) (end 138.2 106.7) (width 0.2) (layer "B.Cu") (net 6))
 (segment (start 137.7 98.4) (end 138.2 97.9) (width 0.2) (layer "B.Cu") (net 6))
 (segment (start 148.5 87.9) (end 150 87.9) (width 0.2) (layer "B.Cu") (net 6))
 (segment (start 164.4125 113.5) (end 157.5625 106.65) (width 0.2) (layer "F.Cu") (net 10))
 (segment (start 158 103.8) (end 159.4375 102.3625) (width 0.2) (layer "F.Cu") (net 10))
 (segment (start 148.6625 96.6) (end 159.4375 96.6) (width 0.2) (layer "F.Cu") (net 10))
 (segment (start 147.5625 95.5) (end 148.6625 96.6) (width 0.2) (layer "F.Cu") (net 10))
 (segment (start 157.5625 105.5) (end 156.625 105.5) (width 0.2) (layer "F.Cu") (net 10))
 (segment (start 159.4375 102.3625) (end 159.4375 95.5) (width 0.2) (layer "F.Cu") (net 10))
 (segment (start 157.5625 106.65) (end 157.5625 105.5) (width 0.2) (layer "F.Cu") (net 10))
 (via (at 156.625 105.5) (size 0.6) (drill 0.3) (layers "F.Cu" "B.Cu") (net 10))
 (via (at 158 103.8) (size 0.6) (drill 0.3) (layers "F.Cu" "B.Cu") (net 10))
 (segment (start 156.625 105.5) (end 158 104.125) (width 0.2) (layer "B.Cu") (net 10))
 (segment (start 158 104.125) (end 158 103.8) (width 0.2) (layer "B.Cu") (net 10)))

